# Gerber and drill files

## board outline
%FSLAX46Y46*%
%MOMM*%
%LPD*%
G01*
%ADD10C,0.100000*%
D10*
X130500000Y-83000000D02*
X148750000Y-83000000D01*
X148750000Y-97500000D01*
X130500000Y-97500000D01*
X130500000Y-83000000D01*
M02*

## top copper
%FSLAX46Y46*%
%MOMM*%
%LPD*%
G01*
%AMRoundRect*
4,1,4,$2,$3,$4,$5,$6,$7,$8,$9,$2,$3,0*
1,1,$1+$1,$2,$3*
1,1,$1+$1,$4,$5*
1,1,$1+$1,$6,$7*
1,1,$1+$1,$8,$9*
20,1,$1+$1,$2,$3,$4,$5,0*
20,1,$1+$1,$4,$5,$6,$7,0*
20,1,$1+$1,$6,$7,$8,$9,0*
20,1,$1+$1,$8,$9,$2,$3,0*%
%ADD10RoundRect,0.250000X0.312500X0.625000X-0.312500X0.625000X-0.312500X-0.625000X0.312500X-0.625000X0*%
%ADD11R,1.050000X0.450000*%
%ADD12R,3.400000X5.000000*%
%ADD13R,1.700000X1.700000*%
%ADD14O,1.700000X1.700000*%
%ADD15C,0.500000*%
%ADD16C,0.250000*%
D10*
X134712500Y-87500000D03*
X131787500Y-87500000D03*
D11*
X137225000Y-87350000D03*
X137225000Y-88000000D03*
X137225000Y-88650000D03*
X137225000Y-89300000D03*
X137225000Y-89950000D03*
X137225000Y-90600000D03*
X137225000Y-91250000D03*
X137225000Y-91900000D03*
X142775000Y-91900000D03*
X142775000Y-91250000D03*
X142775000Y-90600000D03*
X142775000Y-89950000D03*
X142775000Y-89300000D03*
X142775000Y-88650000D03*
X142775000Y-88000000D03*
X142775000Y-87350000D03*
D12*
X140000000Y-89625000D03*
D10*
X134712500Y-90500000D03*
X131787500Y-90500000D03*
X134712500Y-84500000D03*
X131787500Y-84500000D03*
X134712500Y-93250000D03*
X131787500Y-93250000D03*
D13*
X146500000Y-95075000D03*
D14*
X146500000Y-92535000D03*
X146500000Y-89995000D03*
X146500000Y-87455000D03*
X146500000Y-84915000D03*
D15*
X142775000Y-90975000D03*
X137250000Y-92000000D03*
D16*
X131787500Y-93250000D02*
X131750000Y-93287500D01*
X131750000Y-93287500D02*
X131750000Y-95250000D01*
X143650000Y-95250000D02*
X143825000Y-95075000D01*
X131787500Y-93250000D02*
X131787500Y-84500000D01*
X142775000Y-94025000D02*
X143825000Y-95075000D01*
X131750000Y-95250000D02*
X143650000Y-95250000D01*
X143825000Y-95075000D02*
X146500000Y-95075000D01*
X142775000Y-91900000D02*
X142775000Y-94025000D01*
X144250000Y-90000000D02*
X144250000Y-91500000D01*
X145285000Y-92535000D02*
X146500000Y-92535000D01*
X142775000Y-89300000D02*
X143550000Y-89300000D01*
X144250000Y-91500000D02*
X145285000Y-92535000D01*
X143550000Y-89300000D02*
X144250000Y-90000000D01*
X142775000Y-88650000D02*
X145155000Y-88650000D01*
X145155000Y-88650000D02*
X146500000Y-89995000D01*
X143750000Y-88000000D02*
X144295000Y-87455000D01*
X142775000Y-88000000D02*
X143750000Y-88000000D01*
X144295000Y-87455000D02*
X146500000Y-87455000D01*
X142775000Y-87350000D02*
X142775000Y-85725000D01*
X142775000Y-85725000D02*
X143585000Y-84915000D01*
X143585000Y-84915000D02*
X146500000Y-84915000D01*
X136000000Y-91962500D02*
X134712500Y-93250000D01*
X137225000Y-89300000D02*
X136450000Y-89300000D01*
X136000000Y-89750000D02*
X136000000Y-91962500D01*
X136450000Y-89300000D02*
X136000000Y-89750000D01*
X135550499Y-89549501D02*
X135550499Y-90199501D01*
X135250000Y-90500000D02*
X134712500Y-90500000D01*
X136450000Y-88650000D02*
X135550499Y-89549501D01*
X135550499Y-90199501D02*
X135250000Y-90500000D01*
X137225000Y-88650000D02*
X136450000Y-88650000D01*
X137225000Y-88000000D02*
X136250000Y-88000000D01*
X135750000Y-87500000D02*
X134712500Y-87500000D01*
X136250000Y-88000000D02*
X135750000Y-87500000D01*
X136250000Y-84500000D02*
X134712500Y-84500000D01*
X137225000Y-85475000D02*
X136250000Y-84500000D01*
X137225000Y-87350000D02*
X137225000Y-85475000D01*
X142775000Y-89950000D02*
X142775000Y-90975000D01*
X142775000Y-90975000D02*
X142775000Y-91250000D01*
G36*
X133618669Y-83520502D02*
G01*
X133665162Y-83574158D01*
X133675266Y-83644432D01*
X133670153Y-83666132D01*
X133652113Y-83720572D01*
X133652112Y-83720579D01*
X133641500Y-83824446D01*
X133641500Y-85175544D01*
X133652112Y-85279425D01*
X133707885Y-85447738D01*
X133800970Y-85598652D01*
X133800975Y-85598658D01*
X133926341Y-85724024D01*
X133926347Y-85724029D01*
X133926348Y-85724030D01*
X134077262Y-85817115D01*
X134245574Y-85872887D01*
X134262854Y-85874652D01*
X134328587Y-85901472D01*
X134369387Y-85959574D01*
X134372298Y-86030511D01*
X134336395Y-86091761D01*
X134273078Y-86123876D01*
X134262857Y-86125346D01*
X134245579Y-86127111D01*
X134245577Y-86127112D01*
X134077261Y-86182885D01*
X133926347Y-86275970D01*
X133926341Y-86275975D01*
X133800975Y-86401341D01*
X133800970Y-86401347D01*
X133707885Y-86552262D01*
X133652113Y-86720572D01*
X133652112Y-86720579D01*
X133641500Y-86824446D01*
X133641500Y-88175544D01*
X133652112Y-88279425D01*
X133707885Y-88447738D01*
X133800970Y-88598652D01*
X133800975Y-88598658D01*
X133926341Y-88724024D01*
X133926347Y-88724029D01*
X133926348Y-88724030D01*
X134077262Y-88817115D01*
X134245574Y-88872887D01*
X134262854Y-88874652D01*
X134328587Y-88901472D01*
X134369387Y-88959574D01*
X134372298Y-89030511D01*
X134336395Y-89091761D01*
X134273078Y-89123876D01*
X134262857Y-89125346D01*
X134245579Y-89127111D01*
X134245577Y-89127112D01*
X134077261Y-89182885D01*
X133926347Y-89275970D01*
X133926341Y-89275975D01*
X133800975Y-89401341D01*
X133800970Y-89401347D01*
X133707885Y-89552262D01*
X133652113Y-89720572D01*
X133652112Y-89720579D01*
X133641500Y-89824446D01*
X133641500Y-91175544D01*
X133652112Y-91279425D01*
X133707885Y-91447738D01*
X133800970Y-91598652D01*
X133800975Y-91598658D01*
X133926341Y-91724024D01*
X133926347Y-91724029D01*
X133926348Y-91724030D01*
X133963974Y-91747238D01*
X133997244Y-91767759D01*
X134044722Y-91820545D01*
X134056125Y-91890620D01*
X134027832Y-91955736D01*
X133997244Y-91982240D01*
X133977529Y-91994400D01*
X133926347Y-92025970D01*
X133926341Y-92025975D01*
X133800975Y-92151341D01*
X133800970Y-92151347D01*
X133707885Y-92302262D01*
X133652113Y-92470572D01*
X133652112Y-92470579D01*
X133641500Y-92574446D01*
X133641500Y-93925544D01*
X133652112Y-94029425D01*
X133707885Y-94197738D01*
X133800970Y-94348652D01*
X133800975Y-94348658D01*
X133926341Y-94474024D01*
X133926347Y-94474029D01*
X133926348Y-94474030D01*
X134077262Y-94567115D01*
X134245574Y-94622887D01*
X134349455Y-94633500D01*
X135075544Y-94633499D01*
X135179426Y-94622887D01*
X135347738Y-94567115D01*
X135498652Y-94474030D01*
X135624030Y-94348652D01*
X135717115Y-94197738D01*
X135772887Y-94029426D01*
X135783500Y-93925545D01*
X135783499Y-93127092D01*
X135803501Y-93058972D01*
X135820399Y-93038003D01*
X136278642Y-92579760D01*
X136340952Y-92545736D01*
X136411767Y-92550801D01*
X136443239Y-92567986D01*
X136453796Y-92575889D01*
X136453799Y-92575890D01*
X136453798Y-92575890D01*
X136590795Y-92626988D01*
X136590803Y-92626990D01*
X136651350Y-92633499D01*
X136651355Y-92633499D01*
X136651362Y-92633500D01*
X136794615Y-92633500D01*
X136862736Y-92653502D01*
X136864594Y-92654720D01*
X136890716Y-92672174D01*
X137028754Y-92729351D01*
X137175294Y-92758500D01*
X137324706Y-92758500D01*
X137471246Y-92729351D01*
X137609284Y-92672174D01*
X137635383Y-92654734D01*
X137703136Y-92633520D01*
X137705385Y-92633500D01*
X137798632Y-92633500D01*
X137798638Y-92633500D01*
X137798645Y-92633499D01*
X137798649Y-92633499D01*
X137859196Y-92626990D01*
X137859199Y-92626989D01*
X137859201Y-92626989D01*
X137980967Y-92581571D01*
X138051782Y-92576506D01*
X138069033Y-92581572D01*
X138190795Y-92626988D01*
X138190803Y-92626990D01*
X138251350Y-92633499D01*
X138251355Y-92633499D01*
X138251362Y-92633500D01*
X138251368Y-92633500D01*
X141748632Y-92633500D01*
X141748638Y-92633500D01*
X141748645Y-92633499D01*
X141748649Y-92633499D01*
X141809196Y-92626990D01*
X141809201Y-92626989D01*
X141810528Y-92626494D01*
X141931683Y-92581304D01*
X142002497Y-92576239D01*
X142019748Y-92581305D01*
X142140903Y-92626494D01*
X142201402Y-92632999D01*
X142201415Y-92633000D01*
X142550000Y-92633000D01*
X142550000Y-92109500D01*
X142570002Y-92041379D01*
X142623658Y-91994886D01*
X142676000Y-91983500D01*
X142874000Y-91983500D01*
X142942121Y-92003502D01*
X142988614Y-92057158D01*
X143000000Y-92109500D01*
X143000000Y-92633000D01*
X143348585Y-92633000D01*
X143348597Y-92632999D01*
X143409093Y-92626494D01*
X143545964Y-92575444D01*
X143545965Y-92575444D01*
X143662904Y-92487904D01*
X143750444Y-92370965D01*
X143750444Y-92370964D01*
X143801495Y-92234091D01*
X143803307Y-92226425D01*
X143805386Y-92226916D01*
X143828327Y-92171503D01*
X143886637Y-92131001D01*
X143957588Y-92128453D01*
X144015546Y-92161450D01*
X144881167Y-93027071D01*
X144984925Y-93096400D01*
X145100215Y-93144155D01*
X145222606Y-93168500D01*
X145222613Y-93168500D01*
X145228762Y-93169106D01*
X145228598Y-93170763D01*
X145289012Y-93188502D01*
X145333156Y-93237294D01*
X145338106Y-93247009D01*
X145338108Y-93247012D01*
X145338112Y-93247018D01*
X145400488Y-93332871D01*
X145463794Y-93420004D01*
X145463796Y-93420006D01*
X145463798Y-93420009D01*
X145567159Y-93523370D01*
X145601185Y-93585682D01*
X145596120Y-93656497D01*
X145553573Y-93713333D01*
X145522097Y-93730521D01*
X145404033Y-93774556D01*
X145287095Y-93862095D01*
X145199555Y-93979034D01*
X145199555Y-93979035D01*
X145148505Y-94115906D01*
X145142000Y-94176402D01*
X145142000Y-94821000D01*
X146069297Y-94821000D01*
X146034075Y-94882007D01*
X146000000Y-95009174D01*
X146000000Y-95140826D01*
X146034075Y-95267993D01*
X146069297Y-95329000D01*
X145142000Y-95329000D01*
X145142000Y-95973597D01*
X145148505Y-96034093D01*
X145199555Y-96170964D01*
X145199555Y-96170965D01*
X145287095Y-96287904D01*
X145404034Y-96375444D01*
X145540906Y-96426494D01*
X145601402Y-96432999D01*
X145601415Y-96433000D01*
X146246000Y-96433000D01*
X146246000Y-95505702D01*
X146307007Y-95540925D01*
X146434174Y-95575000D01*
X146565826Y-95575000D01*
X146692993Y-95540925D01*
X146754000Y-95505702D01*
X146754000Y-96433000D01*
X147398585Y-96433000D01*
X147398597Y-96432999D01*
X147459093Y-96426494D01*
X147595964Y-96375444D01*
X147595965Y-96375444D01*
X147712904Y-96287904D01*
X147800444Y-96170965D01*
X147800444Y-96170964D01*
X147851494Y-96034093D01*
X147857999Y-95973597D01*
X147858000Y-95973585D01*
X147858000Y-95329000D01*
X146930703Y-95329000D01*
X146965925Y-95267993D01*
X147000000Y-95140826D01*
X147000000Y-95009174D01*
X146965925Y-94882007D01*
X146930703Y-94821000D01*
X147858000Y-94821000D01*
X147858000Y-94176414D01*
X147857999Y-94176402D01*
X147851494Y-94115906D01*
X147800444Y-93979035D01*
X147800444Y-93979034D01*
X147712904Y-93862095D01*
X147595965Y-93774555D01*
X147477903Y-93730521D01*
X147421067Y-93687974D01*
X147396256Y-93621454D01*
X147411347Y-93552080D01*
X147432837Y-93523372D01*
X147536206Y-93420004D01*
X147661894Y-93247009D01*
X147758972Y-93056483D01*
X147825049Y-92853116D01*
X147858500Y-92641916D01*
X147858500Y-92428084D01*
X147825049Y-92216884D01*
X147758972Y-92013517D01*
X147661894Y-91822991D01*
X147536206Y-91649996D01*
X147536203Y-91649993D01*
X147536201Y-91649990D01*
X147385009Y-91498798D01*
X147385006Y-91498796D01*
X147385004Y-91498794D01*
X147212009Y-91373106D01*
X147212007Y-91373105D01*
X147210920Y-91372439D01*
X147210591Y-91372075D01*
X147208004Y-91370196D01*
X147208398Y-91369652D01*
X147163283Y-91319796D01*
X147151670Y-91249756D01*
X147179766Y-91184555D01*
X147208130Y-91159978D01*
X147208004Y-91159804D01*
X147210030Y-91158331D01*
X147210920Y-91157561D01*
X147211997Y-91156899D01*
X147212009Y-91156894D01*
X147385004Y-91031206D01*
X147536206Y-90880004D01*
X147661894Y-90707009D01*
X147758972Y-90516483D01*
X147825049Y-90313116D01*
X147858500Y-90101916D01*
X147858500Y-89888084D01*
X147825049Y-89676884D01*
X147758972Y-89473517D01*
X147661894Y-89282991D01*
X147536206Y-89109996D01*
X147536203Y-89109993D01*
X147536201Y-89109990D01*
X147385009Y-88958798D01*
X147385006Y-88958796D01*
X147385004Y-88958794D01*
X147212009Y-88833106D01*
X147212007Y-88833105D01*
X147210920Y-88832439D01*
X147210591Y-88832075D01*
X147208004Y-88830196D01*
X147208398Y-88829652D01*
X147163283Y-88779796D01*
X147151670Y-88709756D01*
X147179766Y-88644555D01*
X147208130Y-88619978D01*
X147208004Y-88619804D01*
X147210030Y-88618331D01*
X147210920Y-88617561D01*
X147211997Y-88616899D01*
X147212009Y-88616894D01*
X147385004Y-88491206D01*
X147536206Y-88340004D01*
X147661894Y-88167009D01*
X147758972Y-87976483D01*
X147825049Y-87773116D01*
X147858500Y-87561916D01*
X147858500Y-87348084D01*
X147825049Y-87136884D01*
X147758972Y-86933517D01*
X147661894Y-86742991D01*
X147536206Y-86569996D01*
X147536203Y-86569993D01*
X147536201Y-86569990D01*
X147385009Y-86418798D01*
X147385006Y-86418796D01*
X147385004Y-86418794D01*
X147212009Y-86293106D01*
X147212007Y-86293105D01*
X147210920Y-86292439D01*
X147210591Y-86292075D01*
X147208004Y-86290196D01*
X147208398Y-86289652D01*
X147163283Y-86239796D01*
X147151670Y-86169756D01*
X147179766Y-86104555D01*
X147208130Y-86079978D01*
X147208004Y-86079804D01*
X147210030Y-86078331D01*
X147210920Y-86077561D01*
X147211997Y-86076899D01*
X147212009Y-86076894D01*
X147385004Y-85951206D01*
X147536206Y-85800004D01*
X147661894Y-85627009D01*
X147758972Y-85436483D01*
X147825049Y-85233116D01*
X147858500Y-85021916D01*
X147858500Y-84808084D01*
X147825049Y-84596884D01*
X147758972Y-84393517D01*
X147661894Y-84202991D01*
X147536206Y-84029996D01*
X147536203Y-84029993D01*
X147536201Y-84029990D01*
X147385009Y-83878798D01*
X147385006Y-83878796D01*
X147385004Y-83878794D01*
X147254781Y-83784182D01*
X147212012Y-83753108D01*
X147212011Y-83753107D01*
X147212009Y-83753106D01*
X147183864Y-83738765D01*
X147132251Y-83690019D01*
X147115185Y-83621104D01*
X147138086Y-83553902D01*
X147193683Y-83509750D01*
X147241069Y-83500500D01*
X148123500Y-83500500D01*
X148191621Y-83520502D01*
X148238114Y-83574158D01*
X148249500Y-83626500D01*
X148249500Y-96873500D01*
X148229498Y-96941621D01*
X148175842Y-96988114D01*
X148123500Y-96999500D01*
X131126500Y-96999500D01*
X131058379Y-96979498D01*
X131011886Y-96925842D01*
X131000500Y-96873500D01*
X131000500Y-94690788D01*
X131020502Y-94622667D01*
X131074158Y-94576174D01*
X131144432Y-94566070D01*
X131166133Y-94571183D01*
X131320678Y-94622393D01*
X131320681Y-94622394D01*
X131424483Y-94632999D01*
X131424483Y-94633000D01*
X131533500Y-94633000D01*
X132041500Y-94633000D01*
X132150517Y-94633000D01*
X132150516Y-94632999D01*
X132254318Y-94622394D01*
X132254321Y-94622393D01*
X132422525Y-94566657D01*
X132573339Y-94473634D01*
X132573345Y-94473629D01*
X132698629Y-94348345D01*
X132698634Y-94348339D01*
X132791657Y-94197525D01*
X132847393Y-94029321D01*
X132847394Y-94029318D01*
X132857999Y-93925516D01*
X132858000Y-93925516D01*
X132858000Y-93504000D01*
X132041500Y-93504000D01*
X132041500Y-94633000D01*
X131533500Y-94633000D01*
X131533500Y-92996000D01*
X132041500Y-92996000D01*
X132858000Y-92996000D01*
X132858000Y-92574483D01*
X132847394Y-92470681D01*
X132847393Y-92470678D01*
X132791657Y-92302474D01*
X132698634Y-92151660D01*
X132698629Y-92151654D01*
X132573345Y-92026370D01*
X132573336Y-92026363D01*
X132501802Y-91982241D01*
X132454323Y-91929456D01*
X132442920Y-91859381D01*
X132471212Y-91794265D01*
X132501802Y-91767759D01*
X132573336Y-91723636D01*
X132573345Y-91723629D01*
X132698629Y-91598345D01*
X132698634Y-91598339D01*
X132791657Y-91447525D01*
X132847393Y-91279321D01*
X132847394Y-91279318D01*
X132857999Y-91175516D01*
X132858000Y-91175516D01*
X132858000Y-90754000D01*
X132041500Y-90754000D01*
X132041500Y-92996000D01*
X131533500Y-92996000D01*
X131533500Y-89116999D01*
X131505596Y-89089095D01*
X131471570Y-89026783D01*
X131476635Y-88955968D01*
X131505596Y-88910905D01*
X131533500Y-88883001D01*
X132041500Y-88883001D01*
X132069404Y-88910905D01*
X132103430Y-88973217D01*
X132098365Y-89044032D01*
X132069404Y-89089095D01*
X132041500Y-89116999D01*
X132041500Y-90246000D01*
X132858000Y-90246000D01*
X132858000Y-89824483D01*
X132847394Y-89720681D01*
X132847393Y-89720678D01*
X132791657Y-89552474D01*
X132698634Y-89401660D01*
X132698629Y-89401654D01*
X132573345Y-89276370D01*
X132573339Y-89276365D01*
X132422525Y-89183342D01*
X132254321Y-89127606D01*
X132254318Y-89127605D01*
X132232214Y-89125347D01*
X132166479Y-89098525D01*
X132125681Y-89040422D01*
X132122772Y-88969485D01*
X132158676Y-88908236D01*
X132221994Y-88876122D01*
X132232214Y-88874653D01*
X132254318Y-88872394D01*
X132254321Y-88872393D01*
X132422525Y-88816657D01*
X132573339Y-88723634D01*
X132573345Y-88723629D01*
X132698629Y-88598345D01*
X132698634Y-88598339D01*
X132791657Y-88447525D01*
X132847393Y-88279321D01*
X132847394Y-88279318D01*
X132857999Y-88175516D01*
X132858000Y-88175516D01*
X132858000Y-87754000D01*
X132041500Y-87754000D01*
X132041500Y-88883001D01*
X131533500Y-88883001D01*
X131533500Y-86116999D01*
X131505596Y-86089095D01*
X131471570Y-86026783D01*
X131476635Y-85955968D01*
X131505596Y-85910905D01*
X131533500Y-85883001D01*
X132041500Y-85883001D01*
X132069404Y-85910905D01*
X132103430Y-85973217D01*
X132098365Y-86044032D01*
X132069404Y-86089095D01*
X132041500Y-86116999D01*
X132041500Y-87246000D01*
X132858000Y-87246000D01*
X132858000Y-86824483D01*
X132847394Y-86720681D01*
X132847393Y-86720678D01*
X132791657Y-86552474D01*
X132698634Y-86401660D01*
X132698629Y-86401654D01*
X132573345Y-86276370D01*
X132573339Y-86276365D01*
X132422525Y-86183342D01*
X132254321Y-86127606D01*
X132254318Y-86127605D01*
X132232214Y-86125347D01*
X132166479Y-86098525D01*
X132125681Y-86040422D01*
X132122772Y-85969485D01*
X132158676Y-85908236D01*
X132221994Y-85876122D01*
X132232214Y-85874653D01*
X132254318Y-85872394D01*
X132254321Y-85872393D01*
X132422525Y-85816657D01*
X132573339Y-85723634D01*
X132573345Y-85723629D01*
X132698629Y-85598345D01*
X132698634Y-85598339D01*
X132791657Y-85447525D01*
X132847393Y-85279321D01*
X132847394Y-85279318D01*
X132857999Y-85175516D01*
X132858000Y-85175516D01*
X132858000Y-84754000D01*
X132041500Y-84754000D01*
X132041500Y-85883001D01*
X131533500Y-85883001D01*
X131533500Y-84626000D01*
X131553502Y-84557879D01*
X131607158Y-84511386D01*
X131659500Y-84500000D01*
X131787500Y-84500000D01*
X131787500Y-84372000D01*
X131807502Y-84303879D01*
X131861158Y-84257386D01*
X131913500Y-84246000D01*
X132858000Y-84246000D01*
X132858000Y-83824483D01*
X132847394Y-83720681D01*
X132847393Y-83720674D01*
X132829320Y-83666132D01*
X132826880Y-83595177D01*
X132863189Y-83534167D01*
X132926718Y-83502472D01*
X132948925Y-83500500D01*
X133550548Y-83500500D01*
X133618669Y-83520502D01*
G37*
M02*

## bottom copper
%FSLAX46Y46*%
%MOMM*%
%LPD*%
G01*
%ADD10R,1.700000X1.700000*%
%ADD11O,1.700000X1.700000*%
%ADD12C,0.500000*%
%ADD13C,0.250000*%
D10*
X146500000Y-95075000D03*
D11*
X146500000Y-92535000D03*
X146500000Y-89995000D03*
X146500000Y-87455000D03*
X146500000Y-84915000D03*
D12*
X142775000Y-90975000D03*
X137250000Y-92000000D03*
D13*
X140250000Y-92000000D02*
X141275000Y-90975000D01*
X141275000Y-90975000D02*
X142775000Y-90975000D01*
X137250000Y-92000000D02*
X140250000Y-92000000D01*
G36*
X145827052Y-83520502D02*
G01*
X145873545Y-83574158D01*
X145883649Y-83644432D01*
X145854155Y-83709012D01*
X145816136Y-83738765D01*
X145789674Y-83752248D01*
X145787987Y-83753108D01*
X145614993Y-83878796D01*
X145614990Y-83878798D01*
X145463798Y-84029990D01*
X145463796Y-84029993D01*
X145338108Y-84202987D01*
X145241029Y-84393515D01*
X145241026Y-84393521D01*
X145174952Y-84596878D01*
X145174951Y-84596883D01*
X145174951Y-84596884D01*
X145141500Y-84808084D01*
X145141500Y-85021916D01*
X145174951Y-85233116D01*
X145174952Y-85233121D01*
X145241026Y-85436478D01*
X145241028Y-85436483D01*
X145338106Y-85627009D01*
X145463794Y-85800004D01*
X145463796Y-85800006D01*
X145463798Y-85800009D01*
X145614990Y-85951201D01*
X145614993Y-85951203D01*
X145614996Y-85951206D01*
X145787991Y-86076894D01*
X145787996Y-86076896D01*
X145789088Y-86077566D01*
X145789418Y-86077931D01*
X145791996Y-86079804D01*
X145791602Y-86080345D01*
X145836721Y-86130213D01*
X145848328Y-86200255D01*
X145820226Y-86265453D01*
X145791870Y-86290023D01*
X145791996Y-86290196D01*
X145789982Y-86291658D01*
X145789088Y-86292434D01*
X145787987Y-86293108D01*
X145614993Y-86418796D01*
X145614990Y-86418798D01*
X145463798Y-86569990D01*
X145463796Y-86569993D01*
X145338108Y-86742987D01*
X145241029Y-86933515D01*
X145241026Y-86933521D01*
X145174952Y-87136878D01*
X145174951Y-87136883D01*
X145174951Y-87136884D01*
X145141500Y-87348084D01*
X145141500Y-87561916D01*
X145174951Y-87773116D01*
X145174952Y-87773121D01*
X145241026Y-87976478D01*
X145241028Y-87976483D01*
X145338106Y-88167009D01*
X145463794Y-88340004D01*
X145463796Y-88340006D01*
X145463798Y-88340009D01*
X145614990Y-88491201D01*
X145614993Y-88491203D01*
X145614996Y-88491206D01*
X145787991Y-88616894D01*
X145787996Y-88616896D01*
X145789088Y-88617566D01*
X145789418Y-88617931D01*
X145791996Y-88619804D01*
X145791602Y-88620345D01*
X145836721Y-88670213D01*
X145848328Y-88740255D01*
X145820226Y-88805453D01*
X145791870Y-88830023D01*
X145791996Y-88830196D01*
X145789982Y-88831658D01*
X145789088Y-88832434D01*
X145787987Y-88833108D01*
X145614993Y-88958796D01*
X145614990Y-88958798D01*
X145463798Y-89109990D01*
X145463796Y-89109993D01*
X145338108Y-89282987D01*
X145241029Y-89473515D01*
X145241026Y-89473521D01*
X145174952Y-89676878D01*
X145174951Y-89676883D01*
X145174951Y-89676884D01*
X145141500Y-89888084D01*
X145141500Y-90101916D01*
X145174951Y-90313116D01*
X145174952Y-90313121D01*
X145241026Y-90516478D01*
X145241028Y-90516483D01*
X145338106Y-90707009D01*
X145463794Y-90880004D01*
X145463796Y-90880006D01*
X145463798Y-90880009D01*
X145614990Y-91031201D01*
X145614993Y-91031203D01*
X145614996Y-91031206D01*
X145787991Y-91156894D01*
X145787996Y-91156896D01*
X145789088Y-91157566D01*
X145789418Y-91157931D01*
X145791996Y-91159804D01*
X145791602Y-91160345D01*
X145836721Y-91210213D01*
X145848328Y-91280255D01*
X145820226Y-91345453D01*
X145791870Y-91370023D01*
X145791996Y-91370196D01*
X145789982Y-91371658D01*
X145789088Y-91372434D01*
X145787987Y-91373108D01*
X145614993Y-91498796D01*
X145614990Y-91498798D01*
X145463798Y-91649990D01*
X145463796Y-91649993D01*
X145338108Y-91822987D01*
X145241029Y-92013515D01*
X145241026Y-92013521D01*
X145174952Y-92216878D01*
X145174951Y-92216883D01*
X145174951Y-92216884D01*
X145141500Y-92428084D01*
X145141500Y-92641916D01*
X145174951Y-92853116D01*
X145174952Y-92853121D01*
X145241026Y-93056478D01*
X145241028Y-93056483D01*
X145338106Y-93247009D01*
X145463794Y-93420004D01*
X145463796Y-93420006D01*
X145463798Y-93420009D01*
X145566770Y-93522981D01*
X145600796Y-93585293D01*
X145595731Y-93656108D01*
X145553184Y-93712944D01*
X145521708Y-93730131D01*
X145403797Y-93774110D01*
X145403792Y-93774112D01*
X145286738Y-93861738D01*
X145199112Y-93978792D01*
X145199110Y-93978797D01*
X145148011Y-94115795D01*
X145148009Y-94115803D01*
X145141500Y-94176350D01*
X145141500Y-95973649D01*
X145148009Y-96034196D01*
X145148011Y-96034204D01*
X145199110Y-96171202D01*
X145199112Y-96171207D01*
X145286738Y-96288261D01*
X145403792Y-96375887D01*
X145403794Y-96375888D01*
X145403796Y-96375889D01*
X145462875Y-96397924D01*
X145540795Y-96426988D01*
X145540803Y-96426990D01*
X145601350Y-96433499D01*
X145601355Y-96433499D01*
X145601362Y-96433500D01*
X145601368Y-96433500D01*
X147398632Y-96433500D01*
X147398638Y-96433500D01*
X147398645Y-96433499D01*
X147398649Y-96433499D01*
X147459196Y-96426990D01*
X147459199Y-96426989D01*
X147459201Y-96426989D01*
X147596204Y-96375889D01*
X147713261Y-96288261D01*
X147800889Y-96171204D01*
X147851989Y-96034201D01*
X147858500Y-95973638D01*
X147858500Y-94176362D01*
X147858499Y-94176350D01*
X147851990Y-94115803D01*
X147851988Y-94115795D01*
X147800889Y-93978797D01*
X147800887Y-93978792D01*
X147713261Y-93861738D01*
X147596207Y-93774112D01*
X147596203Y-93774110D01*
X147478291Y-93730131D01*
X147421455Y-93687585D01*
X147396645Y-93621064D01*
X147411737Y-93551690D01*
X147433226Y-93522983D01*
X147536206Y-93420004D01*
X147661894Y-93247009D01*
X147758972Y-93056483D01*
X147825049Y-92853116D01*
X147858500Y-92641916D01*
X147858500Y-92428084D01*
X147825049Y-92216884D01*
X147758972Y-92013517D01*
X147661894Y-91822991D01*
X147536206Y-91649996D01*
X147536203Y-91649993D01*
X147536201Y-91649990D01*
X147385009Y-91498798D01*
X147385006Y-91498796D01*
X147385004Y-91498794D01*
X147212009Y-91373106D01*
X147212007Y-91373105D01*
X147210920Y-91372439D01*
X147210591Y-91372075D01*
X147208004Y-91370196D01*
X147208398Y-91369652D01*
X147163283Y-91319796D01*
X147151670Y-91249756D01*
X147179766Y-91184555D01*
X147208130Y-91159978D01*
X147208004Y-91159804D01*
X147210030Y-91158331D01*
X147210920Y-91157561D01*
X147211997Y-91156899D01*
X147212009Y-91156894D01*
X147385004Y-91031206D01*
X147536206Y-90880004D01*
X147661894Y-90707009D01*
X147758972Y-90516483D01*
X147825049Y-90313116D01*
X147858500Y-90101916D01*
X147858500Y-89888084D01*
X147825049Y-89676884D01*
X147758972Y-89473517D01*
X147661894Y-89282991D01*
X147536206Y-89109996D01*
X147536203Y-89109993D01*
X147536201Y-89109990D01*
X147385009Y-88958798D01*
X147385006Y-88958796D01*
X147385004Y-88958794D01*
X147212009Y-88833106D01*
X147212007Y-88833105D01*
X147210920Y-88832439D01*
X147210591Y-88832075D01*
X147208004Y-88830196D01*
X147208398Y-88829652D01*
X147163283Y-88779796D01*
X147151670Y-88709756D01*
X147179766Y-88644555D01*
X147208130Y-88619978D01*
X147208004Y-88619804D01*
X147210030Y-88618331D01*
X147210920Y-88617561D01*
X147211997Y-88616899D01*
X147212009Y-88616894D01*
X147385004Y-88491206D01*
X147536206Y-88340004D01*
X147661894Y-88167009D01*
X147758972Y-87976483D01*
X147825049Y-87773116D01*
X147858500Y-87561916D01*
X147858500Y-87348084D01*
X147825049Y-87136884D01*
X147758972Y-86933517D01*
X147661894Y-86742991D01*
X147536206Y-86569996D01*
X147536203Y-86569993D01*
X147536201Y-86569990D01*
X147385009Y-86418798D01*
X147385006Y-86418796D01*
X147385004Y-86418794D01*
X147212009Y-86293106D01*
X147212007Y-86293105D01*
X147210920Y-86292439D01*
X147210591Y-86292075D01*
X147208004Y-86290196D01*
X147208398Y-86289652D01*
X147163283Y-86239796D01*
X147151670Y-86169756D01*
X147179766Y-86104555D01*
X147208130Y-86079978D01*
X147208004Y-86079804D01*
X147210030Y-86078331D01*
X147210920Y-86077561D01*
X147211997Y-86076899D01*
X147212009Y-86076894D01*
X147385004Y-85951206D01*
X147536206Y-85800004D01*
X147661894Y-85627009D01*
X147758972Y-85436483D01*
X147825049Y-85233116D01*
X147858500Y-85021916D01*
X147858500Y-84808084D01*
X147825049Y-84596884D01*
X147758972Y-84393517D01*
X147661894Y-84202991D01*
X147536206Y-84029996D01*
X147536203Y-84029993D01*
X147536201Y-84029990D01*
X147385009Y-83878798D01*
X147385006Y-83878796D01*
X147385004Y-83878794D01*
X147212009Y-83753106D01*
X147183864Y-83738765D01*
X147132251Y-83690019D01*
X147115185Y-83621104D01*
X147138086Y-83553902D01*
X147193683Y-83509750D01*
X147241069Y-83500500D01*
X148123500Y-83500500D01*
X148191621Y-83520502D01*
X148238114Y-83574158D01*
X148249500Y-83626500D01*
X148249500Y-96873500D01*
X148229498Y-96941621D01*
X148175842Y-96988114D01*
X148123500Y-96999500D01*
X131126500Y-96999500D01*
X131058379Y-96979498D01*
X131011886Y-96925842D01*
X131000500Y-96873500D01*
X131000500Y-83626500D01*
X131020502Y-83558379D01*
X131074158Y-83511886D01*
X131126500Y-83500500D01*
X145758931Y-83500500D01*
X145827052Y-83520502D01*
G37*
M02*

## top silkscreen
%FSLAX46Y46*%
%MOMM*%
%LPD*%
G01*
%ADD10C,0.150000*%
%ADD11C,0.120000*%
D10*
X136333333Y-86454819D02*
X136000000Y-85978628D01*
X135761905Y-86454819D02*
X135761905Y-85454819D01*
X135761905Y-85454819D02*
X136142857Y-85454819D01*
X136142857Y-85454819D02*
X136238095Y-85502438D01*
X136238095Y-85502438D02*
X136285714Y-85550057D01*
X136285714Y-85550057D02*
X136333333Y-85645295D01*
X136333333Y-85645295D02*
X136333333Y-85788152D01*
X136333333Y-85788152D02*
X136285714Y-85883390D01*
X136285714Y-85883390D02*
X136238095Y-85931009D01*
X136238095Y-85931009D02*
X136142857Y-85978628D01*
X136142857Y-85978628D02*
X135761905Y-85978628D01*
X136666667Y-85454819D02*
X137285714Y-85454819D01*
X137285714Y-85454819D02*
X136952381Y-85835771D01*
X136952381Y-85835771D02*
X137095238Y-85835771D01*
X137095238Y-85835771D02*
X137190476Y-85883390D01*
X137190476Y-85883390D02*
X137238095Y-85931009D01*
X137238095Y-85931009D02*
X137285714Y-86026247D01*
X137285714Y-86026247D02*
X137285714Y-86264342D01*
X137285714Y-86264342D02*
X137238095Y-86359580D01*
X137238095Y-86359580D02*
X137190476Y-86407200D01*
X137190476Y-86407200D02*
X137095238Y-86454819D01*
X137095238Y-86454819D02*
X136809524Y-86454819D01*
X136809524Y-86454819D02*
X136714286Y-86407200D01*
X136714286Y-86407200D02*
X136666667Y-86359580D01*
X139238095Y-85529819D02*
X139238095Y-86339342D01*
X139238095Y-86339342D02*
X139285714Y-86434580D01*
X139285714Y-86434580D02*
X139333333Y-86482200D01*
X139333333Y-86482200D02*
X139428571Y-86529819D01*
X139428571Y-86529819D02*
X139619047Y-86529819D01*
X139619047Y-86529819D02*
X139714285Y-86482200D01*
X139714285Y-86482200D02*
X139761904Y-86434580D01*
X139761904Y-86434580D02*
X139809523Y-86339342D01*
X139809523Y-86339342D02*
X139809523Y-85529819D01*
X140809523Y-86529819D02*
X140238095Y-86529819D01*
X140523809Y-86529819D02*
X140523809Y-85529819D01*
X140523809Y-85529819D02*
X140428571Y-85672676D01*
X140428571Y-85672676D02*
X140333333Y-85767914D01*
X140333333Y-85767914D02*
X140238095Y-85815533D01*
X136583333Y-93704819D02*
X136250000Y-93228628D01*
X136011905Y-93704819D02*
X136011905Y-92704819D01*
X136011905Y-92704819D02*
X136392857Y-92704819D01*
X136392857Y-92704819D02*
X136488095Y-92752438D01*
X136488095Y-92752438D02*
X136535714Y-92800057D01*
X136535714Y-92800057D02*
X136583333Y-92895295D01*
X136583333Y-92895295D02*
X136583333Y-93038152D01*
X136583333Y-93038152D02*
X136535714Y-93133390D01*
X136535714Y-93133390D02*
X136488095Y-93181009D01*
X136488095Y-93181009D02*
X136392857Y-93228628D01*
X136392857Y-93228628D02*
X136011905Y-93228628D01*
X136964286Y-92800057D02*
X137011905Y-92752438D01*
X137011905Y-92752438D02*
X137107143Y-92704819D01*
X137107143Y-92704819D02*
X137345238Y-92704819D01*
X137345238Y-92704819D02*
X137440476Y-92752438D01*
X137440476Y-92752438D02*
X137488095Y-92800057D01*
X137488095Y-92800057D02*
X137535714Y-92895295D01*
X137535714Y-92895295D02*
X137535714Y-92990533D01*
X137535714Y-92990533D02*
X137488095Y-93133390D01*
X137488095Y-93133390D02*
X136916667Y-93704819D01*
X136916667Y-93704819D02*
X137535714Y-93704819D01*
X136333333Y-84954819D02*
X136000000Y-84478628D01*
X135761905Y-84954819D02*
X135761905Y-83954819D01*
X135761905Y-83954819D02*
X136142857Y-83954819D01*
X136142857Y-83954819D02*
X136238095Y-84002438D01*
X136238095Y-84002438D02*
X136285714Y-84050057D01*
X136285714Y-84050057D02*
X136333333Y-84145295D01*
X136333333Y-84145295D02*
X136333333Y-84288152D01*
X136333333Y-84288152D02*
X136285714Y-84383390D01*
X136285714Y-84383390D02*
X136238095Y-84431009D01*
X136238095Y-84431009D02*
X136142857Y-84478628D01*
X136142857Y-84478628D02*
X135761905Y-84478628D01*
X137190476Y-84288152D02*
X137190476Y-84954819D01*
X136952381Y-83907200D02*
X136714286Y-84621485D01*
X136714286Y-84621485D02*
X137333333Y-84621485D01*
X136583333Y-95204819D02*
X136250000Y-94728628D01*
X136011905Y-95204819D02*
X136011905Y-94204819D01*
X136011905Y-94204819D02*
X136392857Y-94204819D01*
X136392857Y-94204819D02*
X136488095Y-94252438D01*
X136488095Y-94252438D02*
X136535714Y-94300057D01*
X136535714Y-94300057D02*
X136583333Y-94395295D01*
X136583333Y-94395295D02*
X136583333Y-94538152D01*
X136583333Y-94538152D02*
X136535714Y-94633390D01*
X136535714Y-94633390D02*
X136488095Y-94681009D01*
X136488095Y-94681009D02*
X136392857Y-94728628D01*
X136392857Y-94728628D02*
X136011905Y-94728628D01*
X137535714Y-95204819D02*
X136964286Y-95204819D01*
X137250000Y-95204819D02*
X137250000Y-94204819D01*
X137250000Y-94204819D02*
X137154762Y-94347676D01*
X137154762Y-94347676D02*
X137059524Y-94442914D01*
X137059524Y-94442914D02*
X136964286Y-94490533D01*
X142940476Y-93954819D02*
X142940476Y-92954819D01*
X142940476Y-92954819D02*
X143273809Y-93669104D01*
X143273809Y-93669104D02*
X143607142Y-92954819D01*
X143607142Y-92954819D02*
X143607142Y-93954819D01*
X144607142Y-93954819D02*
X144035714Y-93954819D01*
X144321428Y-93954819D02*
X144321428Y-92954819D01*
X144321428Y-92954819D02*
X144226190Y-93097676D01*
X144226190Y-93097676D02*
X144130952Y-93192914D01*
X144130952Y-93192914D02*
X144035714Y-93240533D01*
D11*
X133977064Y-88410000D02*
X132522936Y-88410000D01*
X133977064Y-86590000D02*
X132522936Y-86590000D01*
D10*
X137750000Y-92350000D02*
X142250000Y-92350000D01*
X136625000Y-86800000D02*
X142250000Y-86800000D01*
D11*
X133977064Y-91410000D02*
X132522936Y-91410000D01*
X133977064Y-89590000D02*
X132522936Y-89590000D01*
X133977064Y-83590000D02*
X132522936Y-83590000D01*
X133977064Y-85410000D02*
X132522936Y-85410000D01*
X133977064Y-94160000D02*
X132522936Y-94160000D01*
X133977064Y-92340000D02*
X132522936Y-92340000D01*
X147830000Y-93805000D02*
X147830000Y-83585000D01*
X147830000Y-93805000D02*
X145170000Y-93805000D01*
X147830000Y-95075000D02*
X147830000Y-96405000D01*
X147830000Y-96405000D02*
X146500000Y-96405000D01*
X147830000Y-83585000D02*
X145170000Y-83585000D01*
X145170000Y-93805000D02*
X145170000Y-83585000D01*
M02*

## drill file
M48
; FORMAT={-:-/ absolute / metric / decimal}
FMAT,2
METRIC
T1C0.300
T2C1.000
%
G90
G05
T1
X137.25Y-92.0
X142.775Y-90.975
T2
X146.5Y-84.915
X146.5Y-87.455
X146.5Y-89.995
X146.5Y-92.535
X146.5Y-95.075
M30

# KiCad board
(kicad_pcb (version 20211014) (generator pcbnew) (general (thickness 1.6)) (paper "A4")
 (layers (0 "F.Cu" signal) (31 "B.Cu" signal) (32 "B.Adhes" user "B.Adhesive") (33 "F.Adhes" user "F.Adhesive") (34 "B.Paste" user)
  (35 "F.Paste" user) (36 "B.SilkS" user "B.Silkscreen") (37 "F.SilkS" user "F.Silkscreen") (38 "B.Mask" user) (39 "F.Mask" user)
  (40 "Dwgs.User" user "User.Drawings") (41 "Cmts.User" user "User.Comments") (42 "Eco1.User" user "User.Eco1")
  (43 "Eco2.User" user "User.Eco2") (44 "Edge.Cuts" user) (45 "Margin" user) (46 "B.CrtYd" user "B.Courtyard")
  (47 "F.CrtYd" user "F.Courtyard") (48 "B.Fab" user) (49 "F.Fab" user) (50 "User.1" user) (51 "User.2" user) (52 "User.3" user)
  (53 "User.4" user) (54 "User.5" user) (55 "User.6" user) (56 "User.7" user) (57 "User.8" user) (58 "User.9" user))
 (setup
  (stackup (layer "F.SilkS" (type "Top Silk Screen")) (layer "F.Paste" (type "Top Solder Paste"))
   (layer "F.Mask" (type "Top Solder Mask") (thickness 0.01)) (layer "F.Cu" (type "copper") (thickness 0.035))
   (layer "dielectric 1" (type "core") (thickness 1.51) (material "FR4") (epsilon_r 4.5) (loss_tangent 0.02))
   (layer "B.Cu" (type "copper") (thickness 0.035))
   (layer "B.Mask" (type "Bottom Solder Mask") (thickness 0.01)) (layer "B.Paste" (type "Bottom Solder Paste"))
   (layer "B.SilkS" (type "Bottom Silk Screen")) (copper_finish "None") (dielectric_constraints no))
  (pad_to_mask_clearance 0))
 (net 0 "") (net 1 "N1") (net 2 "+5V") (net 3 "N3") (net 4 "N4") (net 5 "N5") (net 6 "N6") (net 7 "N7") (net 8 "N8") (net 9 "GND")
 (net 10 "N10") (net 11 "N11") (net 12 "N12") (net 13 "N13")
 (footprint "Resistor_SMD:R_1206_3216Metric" (layer "F.Cu") (at 133.25 87.5 180)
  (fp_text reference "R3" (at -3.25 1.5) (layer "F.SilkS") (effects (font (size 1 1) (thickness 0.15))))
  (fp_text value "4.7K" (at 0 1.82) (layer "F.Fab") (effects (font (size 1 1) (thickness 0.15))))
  (fp_line (start -0.727064 -0.91) (end 0.727064 -0.91) (layer "F.SilkS") (width 0.12))
  (fp_line (start -0.727064 0.91) (end 0.727064 0.91) (layer "F.SilkS") (width 0.12))
  (pad "1" smd roundrect (at -1.4625 0 180) (size 1.125 1.75) (layers "F.Cu" "F.Paste" "F.Mask") (roundrect_rratio 0.2222222222)
   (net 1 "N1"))
  (pad "2" smd roundrect (at 1.4625 0 180) (size 1.125 1.75) (layers "F.Cu" "F.Paste" "F.Mask") (roundrect_rratio 0.2222222222)
   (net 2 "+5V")))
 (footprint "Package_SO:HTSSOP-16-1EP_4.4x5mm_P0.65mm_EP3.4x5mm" (layer "F.Cu") (at 140 89.625)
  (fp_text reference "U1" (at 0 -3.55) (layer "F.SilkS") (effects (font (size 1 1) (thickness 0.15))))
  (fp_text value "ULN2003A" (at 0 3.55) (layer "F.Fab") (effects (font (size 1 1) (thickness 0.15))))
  (fp_line (start -2.25 2.725) (end 2.25 2.725) (layer "F.SilkS") (width 0.15))
  (fp_line (start -3.375 -2.825) (end 2.25 -2.825) (layer "F.SilkS") (width 0.15))
  (pad "" smd rect (at 1.1334 -1.875) (size 0.88 1.05) (layers "F.Paste"))
  (pad "" smd rect (at 0 1.875) (size 0.88 1.05) (layers "F.Paste"))
  (pad "" smd rect (at 0 -0.625) (size 0.88 1.05) (layers "F.Paste"))
  (pad "" smd rect (at 1.1334 -0.625) (size 0.88 1.05) (layers "F.Paste"))
  (pad "" smd rect (at -1.1334 -1.875) (size 0.88 1.05) (layers "F.Paste"))
  (pad "" smd rect (at -1.1334 1.875) (size 0.88 1.05) (layers "F.Paste"))
  (pad "" smd rect (at 1.1334 0.625) (size 0.88 1.05) (layers "F.Paste"))
  (pad "" smd rect (at -1.1334 0.625) (size 0.88 1.05) (layers "F.Paste"))
  (pad "" smd rect (at 0 0.625) (size 0.88 1.05) (layers "F.Paste"))
  (pad "" smd rect (at 0 -1.875) (size 0.88 1.05) (layers "F.Paste"))
  (pad "" smd rect (at 1.1334 1.875) (size 0.88 1.05) (layers "F.Paste"))
  (pad "" smd rect (at -1.1334 -0.625) (size 0.88 1.05) (layers "F.Paste"))
  (pad "1" smd rect (at -2.775 -2.275) (size 1.05 0.45) (layers "F.Cu" "F.Paste" "F.Mask") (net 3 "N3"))
  (pad "2" smd rect (at -2.775 -1.625) (size 1.05 0.45) (layers "F.Cu" "F.Paste" "F.Mask") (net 1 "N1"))
  (pad "3" smd rect (at -2.775 -0.975) (size 1.05 0.45) (layers "F.Cu" "F.Paste" "F.Mask") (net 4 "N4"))
  (pad "4" smd rect (at -2.775 -0.325) (size 1.05 0.45) (layers "F.Cu" "F.Paste" "F.Mask") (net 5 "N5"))
  (pad "5" smd rect (at -2.775 0.325) (size 1.05 0.45) (layers "F.Cu" "F.Paste" "F.Mask") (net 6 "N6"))
  (pad "6" smd rect (at -2.775 0.975) (size 1.05 0.45) (layers "F.Cu" "F.Paste" "F.Mask") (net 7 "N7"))
  (pad "7" smd rect (at -2.775 1.625) (size 1.05 0.45) (layers "F.Cu" "F.Paste" "F.Mask") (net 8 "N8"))
  (pad "8" smd rect (at -2.775 2.275) (size 1.05 0.45) (layers "F.Cu" "F.Paste" "F.Mask") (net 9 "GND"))
  (pad "9" smd rect (at 2.775 2.275) (size 1.05 0.45) (layers "F.Cu" "F.Paste" "F.Mask") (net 2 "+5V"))
  (pad "10" smd rect (at 2.775 1.625) (size 1.05 0.45) (layers "F.Cu" "F.Paste" "F.Mask") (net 9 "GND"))
  (pad "11" smd rect (at 2.775 0.975) (size 1.05 0.45) (layers "F.Cu" "F.Paste" "F.Mask") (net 9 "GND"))
  (pad "12" smd rect (at 2.775 0.325) (size 1.05 0.45) (layers "F.Cu" "F.Paste" "F.Mask") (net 9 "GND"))
  (pad "13" smd rect (at 2.775 -0.325) (size 1.05 0.45) (layers "F.Cu" "F.Paste" "F.Mask") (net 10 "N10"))
  (pad "14" smd rect (at 2.775 -0.975) (size 1.05 0.45) (layers "F.Cu" "F.Paste" "F.Mask") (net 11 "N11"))
  (pad "15" smd rect (at 2.775 -1.625) (size 1.05 0.45) (layers "F.Cu" "F.Paste" "F.Mask") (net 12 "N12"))
  (pad "16" smd rect (at 2.775 -2.275) (size 1.05 0.45) (layers "F.Cu" "F.Paste" "F.Mask") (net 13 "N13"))
  (pad "17" smd rect (at 0 0) (size 3.4 5) (layers "F.Cu" "F.Mask")))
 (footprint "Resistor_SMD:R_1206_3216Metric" (layer "F.Cu") (at 133.25 90.5 180)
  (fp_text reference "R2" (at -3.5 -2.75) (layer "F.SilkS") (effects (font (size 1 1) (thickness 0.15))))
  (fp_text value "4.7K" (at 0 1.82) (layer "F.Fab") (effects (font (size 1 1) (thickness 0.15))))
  (fp_line (start -0.727064 -0.91) (end 0.727064 -0.91) (layer "F.SilkS") (width 0.12))
  (fp_line (start -0.727064 0.91) (end 0.727064 0.91) (layer "F.SilkS") (width 0.12))
  (pad "1" smd roundrect (at -1.4625 0 180) (size 1.125 1.75) (layers "F.Cu" "F.Paste" "F.Mask") (roundrect_rratio 0.2222222222)
   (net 4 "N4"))
  (pad "2" smd roundrect (at 1.4625 0 180) (size 1.125 1.75) (layers "F.Cu" "F.Paste" "F.Mask") (roundrect_rratio 0.2222222222)
   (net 2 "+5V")))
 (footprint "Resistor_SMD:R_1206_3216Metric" (layer "F.Cu") (at 133.25 84.5 180)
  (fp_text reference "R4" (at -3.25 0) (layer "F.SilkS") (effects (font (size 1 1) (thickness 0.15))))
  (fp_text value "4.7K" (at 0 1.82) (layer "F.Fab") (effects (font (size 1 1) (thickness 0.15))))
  (fp_line (start -0.727064 0.91) (end 0.727064 0.91) (layer "F.SilkS") (width 0.12))
  (fp_line (start -0.727064 -0.91) (end 0.727064 -0.91) (layer "F.SilkS") (width 0.12))
  (pad "1" smd roundrect (at -1.4625 0 180) (size 1.125 1.75) (layers "F.Cu" "F.Paste" "F.Mask") (roundrect_rratio 0.2222222222)
   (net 3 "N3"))
  (pad "2" smd roundrect (at 1.4625 0 180) (size 1.125 1.75) (layers "F.Cu" "F.Paste" "F.Mask") (roundrect_rratio 0.2222222222)
   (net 2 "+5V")))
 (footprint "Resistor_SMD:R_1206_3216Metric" (layer "F.Cu") (at 133.25 93.25 180)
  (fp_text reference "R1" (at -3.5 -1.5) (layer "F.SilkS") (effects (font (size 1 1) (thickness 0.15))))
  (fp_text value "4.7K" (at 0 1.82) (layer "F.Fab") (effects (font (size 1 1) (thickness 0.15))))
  (fp_line (start -0.727064 -0.91) (end 0.727064 -0.91) (layer "F.SilkS") (width 0.12))
  (fp_line (start -0.727064 0.91) (end 0.727064 0.91) (layer "F.SilkS") (width 0.12))
  (pad "1" smd roundrect (at -1.4625 0 180) (size 1.125 1.75) (layers "F.Cu" "F.Paste" "F.Mask") (roundrect_rratio 0.2222222222)
   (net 5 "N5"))
  (pad "2" smd roundrect (at 1.4625 0 180) (size 1.125 1.75) (layers "F.Cu" "F.Paste" "F.Mask") (roundrect_rratio 0.2222222222)
   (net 2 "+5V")))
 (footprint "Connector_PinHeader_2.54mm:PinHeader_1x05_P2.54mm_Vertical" (layer "F.Cu") (at 146.5 95.075 180)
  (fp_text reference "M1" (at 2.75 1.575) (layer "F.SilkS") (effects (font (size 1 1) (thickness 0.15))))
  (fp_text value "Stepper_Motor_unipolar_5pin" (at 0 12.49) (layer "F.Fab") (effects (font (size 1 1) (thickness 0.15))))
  (fp_line (start -1.33 1.27) (end -1.33 11.49) (layer "F.SilkS") (width 0.12))
  (fp_line (start -1.33 1.27) (end 1.33 1.27) (layer "F.SilkS") (width 0.12))
  (fp_line (start -1.33 0) (end -1.33 -1.33) (layer "F.SilkS") (width 0.12))
  (fp_line (start -1.33 -1.33) (end 0 -1.33) (layer "F.SilkS") (width 0.12))
  (fp_line (start -1.33 11.49) (end 1.33 11.49) (layer "F.SilkS") (width 0.12))
  (fp_line (start 1.33 1.27) (end 1.33 11.49) (layer "F.SilkS") (width 0.12))
  (pad "1" thru_hole rect (at 0 0 180) (size 1.7 1.7) (drill 1) (layers *.Cu *.Mask) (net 2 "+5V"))
  (pad "2" thru_hole oval (at 0 2.54 180) (size 1.7 1.7) (drill 1) (layers *.Cu *.Mask) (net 10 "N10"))
  (pad "3" thru_hole oval (at 0 5.08 180) (size 1.7 1.7) (drill 1) (layers *.Cu *.Mask) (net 11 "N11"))
  (pad "4" thru_hole oval (at 0 7.62 180) (size 1.7 1.7) (drill 1) (layers *.Cu *.Mask) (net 12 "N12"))
  (pad "5" thru_hole oval (at 0 10.16 180) (size 1.7 1.7) (drill 1) (layers *.Cu *.Mask) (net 13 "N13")))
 (gr_rect (start 130.5 83) (end 148.75 97.5) (layer "Edge.Cuts") (width 0.1) (fill none))
 (segment (start 131.7875 93.25) (end 131.75 93.2875) (width 0.25) (layer "F.Cu") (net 2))
 (segment (start 131.75 93.2875) (end 131.75 95.25) (width 0.25) (layer "F.Cu") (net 2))
 (segment (start 143.65 95.25) (end 143.825 95.075) (width 0.25) (layer "F.Cu") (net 2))
 (segment (start 131.7875 93.25) (end 131.7875 84.5) (width 0.25) (layer "F.Cu") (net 2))
 (segment (start 142.775 94.025) (end 143.825 95.075) (width 0.25) (layer "F.Cu") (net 2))
 (segment (start 131.75 95.25) (end 143.65 95.25) (width 0.25) (layer "F.Cu") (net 2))
 (segment (start 143.825 95.075) (end 146.5 95.075) (width 0.25) (layer "F.Cu") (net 2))
 (segment (start 142.775 91.9) (end 142.775 94.025) (width 0.25) (layer "F.Cu") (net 2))
 (segment (start 144.25 90) (end 144.25 91.5) (width 0.25) (layer "F.Cu") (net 10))
 (segment (start 145.285 92.535) (end 146.5 92.535) (width 0.25) (layer "F.Cu") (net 10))
 (segment (start 142.775 89.3) (end 143.55 89.3) (width 0.25) (layer "F.Cu") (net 10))
 (segment (start 144.25 91.5) (end 145.285 92.535) (width 0.25) (layer "F.Cu") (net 10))
 (segment (start 143.55 89.3) (end 144.25 90) (width 0.25) (layer "F.Cu") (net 10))
 (segment (start 142.775 88.65) (end 145.155 88.65) (width 0.25) (layer "F.Cu") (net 11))
 (segment (start 145.155 88.65) (end 146.5 89.995) (width 0.25) (layer "F.Cu") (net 11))
 (segment (start 143.75 88) (end 144.295 87.455) (width 0.25) (layer "F.Cu") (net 12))
 (segment (start 142.775 88) (end 143.75 88) (width 0.25) (layer "F.Cu") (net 12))
 (segment (start 144.295 87.455) (end 146.5 87.455) (width 0.25) (layer "F.Cu") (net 12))
 (segment (start 142.775 87.35) (end 142.775 85.725) (width 0.25) (layer "F.Cu") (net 13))
 (segment (start 142.775 85.725) (end 143.585 84.915) (width 0.25) (layer "F.Cu") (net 13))
 (segment (start 143.585 84.915) (end 146.5 84.915) (width 0.25) (layer "F.Cu") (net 13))
 (segment (start 136 91.9625) (end 134.7125 93.25) (width 0.25) (layer "F.Cu") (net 5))
 (segment (start 137.225 89.3) (end 136.45 89.3) (width 0.25) (layer "F.Cu") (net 5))
 (segment (start 136 89.75) (end 136 91.9625) (width 0.25) (layer "F.Cu") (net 5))
 (segment (start 136.45 89.3) (end 136 89.75) (width 0.25) (layer "F.Cu") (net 5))
 (segment (start 135.550499 89.549501) (end 135.550499 90.199501) (width 0.25) (layer "F.Cu") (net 4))
 (segment (start 135.25 90.5) (end 134.7125 90.5) (width 0.25) (layer "F.Cu") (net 4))
 (segment (start 136.45 88.65) (end 135.550499 89.549501) (width 0.25) (layer "F.Cu") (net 4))
 (segment (start 135.550499 90.199501) (end 135.25 90.5) (width 0.25) (layer "F.Cu") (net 4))
 (segment (start 137.225 88.65) (end 136.45 88.65) (width 0.25) (layer "F.Cu") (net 4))
 (segment (start 137.225 88) (end 136.25 88) (width 0.25) (layer "F.Cu") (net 1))
 (segment (start 135.75 87.5) (end 134.7125 87.5) (width 0.25) (layer "F.Cu") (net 1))
 (segment (start 136.25 88) (end 135.75 87.5) (width 0.25) (layer "F.Cu") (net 1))
 (segment (start 136.25 84.5) (end 134.7125 84.5) (width 0.25) (layer "F.Cu") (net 3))
 (segment (start 137.225 85.475) (end 136.25 84.5) (width 0.25) (layer "F.Cu") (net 3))
 (segment (start 137.225 87.35) (end 137.225 85.475) (width 0.25) (layer "F.Cu") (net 3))
 (segment (start 142.775 89.95) (end 142.775 90.975) (width 0.25) (layer "F.Cu") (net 9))
 (segment (start 142.775 90.975) (end 142.775 91.25) (width 0.25) (layer "F.Cu") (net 9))
 (via (at 142.775 90.975) (size 0.5) (drill 0.3) (layers "F.Cu" "B.Cu") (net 9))
 (via (at 137.25 92) (size 0.5) (drill 0.3) (layers "F.Cu" "B.Cu") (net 9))
 (segment (start 140.25 92) (end 141.275 90.975) (width 0.25) (layer "B.Cu") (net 9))
 (segment (start 141.275 90.975) (end 142.775 90.975) (width 0.25) (layer "B.Cu") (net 9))
 (segment (start 137.25 92) (end 140.25 92) (width 0.25) (layer "B.Cu") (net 9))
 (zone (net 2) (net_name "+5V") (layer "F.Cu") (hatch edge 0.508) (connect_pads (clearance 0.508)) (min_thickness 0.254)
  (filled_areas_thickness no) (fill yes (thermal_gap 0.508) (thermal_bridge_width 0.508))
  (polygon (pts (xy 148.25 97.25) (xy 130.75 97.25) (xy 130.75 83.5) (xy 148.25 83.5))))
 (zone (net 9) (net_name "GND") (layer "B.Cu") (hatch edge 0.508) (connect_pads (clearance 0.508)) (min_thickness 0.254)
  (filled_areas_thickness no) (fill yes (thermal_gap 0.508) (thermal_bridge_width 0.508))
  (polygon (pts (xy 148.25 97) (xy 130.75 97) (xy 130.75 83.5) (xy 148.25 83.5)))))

